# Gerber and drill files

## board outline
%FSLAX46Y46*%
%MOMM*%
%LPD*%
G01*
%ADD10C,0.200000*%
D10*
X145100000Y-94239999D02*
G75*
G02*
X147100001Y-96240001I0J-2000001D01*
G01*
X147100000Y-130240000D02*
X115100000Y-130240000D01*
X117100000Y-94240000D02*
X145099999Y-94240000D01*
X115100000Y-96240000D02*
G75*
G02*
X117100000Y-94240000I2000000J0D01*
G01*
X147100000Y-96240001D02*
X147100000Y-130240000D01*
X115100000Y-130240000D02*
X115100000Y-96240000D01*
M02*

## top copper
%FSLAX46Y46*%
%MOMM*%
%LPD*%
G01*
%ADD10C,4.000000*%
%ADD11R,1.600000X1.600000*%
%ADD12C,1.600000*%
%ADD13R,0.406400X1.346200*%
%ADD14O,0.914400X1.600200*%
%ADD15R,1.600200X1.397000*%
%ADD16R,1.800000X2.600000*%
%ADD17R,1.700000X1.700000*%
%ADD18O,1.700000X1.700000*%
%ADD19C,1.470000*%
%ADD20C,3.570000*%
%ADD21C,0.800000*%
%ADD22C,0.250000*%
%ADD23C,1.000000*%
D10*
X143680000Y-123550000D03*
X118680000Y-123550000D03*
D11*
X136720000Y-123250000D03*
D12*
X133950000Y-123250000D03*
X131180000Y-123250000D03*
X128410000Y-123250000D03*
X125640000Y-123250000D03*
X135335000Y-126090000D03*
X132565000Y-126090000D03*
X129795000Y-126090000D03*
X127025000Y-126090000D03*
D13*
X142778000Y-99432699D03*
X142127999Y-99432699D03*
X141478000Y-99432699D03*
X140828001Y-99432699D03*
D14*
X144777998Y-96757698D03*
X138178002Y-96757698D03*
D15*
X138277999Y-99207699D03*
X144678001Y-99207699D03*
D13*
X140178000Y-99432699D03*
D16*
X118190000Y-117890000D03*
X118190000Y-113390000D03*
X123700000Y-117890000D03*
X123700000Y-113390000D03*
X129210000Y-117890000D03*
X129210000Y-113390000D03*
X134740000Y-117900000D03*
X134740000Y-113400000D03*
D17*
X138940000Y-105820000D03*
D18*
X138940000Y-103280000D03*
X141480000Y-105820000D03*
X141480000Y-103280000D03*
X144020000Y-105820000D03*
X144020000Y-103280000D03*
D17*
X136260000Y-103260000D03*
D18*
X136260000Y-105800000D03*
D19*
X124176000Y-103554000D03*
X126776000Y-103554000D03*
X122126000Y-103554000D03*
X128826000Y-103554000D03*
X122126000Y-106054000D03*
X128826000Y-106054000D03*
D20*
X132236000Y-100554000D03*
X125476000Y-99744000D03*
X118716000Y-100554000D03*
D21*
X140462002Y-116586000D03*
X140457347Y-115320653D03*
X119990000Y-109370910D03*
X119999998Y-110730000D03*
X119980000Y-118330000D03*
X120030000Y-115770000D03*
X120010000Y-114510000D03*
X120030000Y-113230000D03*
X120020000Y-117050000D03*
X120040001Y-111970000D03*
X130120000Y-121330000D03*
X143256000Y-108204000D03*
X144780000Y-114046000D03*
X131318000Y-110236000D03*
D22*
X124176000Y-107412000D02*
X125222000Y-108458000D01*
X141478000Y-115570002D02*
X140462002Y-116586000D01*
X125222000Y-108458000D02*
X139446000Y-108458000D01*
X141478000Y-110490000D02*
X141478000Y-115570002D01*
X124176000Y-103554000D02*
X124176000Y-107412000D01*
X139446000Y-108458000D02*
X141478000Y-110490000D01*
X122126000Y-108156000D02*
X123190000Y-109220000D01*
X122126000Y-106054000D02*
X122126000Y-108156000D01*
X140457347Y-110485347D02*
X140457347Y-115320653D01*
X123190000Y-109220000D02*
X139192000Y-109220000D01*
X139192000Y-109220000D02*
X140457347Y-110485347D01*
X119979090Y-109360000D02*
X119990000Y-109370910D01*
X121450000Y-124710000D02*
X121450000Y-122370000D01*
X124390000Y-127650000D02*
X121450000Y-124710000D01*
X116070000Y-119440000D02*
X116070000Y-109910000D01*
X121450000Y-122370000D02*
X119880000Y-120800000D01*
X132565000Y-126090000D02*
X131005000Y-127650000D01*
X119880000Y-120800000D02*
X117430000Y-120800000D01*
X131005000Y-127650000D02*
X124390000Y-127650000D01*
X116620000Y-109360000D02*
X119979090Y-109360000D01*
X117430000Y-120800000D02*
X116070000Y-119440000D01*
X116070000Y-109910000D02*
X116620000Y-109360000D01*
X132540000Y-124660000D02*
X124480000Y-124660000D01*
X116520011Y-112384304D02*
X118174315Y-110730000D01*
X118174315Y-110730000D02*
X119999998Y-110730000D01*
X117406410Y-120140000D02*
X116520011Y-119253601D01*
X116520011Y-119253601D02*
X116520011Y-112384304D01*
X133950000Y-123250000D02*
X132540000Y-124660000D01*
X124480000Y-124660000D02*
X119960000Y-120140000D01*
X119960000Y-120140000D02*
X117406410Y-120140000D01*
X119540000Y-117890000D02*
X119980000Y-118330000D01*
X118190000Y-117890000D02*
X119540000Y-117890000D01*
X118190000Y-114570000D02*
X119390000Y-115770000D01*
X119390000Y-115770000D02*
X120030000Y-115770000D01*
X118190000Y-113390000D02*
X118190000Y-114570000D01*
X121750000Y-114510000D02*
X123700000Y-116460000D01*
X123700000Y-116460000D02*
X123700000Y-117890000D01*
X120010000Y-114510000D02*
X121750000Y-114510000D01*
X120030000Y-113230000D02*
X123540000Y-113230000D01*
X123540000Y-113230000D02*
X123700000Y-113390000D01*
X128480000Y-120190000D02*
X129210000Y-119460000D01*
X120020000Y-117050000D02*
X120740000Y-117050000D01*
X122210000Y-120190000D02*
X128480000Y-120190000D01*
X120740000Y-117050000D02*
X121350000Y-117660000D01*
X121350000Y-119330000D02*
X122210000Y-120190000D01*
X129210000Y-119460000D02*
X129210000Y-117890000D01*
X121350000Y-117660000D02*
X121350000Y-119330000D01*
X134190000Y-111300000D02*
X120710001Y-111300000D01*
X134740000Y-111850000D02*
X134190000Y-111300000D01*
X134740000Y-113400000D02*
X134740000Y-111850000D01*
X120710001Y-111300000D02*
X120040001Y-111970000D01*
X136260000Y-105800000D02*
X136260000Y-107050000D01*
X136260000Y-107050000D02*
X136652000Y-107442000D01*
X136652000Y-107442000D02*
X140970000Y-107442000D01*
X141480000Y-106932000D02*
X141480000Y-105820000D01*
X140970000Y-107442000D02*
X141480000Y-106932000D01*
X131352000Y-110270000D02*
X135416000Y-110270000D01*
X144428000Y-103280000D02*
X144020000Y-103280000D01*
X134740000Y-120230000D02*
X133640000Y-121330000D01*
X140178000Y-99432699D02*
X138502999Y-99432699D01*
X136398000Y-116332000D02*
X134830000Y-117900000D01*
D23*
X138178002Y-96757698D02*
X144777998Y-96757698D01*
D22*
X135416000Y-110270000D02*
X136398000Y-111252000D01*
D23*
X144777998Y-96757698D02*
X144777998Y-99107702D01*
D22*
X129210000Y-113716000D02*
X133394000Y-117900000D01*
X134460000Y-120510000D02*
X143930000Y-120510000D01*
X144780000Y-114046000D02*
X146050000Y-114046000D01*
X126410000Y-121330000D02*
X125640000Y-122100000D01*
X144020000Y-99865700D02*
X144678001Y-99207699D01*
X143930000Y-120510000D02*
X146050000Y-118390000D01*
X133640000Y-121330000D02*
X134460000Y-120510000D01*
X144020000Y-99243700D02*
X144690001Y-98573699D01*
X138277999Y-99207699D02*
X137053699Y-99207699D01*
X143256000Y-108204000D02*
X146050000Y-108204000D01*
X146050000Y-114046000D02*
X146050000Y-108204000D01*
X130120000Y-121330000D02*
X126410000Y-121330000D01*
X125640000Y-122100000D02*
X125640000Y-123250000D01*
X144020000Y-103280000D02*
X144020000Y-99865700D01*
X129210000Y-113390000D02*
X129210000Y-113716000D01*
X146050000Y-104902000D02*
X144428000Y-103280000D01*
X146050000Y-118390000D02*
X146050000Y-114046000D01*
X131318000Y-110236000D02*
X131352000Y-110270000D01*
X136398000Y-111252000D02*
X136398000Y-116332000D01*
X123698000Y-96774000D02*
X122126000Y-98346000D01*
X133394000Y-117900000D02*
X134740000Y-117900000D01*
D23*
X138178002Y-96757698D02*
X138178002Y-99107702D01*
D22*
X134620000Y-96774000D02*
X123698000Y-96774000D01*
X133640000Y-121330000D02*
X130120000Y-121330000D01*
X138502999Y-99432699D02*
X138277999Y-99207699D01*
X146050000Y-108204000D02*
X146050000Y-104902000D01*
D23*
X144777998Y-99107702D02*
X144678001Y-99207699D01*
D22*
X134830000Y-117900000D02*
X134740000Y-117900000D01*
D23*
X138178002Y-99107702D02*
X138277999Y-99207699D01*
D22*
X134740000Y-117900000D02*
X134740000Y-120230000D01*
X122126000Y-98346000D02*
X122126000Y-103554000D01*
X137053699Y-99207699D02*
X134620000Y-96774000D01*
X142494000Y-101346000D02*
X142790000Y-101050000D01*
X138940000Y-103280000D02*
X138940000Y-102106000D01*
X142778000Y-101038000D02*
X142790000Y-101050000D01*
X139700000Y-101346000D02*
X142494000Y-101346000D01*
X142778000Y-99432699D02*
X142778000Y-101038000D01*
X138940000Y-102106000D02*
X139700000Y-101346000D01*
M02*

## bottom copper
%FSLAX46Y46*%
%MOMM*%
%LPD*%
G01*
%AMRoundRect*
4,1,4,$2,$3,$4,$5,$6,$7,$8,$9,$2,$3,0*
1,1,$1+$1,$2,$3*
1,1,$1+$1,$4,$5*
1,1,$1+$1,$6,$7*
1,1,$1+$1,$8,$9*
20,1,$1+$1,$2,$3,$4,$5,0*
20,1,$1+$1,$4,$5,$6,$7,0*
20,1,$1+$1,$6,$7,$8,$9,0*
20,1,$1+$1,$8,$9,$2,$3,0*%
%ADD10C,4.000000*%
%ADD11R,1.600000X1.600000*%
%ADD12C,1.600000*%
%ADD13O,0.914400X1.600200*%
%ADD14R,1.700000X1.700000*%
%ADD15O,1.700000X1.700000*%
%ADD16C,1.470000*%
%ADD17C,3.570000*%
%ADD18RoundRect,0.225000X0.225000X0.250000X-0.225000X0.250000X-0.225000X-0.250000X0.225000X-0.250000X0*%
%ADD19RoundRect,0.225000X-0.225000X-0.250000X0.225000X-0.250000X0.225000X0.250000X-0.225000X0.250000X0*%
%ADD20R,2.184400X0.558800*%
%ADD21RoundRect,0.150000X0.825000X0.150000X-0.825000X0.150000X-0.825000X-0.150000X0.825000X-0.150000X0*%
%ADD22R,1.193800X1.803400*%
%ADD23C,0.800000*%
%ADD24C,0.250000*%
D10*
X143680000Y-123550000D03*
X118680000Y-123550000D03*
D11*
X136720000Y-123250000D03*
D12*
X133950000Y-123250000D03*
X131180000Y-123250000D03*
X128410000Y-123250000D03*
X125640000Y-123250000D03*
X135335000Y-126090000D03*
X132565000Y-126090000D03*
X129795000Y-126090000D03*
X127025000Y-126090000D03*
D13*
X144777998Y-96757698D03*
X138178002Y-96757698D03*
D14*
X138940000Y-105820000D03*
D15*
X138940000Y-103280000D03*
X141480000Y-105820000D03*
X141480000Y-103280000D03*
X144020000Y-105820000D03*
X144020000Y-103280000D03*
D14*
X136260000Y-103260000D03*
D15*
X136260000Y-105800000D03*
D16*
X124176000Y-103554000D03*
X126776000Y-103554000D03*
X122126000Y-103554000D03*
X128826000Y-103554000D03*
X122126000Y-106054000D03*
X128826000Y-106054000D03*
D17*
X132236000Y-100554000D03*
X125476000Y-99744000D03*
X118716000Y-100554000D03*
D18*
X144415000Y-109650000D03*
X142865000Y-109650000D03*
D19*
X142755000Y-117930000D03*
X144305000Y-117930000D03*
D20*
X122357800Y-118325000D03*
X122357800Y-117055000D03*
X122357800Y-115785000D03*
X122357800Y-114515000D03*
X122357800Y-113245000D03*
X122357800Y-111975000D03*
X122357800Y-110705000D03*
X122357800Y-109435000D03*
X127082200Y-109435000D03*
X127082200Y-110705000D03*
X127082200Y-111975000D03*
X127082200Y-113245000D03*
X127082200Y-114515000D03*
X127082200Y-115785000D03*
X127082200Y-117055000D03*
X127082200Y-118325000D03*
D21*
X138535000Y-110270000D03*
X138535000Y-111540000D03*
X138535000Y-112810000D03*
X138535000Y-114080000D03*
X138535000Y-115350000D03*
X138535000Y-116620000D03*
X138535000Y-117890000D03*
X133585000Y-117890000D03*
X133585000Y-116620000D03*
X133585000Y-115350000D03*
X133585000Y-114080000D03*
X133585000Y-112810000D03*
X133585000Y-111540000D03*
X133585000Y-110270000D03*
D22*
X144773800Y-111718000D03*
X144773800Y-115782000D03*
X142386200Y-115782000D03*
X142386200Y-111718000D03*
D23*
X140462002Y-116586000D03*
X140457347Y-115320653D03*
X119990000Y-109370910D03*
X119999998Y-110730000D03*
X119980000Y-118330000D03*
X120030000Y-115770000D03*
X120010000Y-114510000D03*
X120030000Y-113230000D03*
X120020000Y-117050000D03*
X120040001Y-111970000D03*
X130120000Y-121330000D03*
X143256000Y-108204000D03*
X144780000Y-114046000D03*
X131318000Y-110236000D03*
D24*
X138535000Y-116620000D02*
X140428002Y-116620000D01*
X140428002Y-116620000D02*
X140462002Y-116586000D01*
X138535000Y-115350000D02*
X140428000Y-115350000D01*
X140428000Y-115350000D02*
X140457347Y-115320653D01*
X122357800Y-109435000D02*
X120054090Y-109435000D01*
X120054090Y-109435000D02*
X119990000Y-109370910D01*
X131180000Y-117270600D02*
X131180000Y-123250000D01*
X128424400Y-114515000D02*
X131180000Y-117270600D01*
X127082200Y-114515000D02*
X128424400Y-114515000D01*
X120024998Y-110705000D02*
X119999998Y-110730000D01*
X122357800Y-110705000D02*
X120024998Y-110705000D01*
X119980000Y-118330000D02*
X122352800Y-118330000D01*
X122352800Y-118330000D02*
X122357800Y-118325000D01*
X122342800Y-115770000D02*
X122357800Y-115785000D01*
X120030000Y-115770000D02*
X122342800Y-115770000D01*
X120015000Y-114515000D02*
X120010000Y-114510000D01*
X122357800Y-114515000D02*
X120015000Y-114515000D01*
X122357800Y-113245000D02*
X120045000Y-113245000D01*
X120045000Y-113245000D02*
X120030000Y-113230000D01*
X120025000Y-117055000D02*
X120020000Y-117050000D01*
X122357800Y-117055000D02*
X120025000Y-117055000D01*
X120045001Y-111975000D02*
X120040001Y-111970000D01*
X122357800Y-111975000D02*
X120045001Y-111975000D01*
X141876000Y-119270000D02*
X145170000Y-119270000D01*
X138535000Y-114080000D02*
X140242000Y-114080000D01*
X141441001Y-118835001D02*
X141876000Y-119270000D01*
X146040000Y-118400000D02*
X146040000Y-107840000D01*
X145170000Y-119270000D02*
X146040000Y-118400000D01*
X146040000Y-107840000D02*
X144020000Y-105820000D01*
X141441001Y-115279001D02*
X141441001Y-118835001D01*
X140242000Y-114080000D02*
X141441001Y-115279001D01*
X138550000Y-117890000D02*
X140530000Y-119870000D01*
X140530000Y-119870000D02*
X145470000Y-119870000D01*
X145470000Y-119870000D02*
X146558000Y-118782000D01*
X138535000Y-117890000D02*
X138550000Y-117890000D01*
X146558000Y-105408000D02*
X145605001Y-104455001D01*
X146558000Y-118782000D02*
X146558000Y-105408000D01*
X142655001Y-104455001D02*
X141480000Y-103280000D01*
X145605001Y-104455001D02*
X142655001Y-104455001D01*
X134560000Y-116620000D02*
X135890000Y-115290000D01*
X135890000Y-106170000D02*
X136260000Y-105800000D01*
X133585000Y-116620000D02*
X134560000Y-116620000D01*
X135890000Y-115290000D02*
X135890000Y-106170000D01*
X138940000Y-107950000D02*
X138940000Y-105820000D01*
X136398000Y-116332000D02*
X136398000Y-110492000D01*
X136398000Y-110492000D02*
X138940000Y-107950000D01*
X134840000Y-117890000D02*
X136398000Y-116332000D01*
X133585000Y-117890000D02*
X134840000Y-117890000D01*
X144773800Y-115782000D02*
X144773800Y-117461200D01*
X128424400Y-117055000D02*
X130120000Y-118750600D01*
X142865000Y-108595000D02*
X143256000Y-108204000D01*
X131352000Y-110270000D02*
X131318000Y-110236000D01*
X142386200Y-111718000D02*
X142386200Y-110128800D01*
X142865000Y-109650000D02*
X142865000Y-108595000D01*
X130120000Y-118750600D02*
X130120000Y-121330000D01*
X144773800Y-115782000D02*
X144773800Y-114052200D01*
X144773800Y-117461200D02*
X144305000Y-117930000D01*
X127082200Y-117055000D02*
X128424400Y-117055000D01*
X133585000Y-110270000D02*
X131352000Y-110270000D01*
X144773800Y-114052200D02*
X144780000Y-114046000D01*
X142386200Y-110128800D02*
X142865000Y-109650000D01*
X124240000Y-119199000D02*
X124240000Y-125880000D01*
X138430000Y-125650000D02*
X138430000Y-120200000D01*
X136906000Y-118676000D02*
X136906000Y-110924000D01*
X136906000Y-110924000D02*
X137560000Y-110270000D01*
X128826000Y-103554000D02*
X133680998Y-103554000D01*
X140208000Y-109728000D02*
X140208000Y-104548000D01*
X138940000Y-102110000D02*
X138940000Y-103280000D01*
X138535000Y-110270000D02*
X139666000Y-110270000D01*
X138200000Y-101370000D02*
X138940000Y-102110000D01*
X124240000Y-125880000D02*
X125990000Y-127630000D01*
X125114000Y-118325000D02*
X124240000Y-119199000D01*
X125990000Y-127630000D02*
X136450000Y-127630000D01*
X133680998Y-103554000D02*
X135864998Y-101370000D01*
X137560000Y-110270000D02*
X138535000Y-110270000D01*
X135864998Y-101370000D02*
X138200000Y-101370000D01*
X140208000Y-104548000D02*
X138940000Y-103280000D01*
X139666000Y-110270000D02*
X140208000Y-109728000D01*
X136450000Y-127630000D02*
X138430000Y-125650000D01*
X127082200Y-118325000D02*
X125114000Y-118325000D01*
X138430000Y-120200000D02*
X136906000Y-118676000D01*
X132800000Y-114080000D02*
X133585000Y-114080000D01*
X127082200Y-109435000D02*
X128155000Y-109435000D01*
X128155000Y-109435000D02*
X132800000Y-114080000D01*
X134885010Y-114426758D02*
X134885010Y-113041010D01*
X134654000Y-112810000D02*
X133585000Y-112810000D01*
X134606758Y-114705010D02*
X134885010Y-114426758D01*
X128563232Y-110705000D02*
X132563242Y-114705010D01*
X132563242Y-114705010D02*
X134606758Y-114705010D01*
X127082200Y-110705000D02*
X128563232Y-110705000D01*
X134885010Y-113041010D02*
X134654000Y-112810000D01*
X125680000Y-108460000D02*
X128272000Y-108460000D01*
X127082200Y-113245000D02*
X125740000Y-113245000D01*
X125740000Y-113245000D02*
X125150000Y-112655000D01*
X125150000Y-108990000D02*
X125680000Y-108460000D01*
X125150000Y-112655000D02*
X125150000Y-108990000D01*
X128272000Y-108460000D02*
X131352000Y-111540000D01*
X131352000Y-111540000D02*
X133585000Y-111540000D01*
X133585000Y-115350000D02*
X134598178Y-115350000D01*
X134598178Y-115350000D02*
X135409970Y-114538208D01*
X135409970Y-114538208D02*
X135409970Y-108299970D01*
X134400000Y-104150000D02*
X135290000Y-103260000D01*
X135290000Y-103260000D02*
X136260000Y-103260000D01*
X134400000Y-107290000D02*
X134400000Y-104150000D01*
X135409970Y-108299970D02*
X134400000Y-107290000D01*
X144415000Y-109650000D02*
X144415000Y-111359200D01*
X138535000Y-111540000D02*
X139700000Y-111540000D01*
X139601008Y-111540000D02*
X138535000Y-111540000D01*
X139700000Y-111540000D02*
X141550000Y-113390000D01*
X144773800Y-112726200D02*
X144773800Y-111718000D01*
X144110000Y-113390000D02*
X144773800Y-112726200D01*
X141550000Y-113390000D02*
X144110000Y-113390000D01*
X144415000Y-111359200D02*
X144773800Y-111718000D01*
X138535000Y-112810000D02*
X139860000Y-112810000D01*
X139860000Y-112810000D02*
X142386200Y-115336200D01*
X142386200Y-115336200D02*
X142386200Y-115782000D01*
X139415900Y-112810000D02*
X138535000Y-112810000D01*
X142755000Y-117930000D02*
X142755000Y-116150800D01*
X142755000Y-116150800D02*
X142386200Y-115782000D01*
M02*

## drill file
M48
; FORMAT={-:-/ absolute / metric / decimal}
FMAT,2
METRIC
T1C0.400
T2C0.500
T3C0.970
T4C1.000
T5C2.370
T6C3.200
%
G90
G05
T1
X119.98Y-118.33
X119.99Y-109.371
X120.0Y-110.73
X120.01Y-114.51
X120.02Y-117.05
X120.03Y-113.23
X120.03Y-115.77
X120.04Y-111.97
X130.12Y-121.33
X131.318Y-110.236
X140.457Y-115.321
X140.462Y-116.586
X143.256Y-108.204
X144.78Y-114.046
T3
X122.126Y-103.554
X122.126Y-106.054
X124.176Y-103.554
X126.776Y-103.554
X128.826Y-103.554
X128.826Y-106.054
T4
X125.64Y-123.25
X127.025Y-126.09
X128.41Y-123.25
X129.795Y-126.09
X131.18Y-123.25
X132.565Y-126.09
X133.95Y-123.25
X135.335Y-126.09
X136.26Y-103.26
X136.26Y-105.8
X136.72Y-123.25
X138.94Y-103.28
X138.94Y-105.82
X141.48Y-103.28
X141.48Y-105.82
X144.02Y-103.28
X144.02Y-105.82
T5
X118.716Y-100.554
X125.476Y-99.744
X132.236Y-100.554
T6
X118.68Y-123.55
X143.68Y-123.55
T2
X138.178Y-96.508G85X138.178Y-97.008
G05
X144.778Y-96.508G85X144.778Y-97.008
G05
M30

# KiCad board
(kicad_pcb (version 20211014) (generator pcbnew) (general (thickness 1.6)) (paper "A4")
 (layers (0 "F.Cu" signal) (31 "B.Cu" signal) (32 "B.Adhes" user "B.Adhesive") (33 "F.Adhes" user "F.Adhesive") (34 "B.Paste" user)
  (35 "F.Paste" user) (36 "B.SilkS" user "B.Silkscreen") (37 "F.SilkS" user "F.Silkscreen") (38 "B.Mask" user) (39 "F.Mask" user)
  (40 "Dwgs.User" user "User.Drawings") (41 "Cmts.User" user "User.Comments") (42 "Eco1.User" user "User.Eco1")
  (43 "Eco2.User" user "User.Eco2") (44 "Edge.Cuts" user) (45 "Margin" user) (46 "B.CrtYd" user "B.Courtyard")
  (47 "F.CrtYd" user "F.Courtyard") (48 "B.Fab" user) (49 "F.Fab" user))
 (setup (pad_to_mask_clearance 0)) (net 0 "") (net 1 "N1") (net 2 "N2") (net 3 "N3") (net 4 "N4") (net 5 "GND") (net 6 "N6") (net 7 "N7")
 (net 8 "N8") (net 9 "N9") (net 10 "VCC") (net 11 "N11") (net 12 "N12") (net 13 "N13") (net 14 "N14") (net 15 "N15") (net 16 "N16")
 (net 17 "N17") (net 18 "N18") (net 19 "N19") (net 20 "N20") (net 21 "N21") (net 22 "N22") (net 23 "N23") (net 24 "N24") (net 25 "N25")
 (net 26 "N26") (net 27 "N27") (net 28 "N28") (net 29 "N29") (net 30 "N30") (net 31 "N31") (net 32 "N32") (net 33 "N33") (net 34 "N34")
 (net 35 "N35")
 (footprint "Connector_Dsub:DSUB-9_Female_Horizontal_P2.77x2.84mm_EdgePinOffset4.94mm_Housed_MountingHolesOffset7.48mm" (layer "F.Cu")
  (at 136.72 123.25)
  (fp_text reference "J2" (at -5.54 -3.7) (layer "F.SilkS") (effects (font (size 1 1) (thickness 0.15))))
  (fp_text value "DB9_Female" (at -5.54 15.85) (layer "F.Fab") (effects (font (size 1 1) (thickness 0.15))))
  (pad "0" thru_hole circle locked (at 6.96 0.3) (size 4 4) (drill 3.2) (layers *.Cu *.Mask))
  (pad "0" thru_hole circle locked (at -18.04 0.3) (size 4 4) (drill 3.2) (layers *.Cu *.Mask))
  (pad "1" thru_hole rect locked (at 0 0) (size 1.6 1.6) (drill 1) (layers *.Cu *.Mask) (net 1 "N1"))
  (pad "2" thru_hole circle locked (at -2.77 0) (size 1.6 1.6) (drill 1) (layers *.Cu *.Mask) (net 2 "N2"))
  (pad "3" thru_hole circle locked (at -5.54 0) (size 1.6 1.6) (drill 1) (layers *.Cu *.Mask) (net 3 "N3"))
  (pad "4" thru_hole circle locked (at -8.31 0) (size 1.6 1.6) (drill 1) (layers *.Cu *.Mask) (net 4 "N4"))
  (pad "5" thru_hole circle locked (at -11.08 0) (size 1.6 1.6) (drill 1) (layers *.Cu *.Mask) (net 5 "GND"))
  (pad "6" thru_hole circle locked (at -1.385 2.84) (size 1.6 1.6) (drill 1) (layers *.Cu *.Mask) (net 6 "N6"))
  (pad "7" thru_hole circle locked (at -4.155 2.84) (size 1.6 1.6) (drill 1) (layers *.Cu *.Mask) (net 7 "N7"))
  (pad "8" thru_hole circle locked (at -6.925 2.84) (size 1.6 1.6) (drill 1) (layers *.Cu *.Mask) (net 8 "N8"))
  (pad "9" thru_hole circle locked (at -9.695 2.84) (size 1.6 1.6) (drill 1) (layers *.Cu *.Mask) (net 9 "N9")))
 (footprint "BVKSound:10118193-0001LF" (layer "F.Cu") (at 141.478 96.774 180)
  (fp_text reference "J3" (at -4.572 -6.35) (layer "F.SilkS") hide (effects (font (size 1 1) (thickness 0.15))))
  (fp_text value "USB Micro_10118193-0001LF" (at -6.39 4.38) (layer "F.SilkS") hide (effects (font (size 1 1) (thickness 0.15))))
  (pad "1" smd rect locked (at -1.3 -2.658699 180) (size 0.4064 1.3462) (layers "F.Cu" "F.Paste" "F.Mask") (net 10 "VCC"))
  (pad "2" smd rect locked (at -0.649999 -2.658699 180) (size 0.4064 1.3462) (layers "F.Cu" "F.Paste" "F.Mask") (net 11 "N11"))
  (pad "3" smd rect locked (at 0 -2.658699 180) (size 0.4064 1.3462) (layers "F.Cu" "F.Paste" "F.Mask") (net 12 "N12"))
  (pad "4" smd rect locked (at 0.649999 -2.658699 180) (size 0.4064 1.3462) (layers "F.Cu" "F.Paste" "F.Mask") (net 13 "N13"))
  (pad "5" thru_hole oval locked (at -3.299998 0.016302 270) (size 1.6002 0.9144) (drill oval 1 0.5) (layers *.Cu *.Mask) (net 5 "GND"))
  (pad "5" thru_hole oval locked (at 3.299998 0.016302 270) (size 1.6002 0.9144) (drill oval 1 0.5) (layers *.Cu *.Mask) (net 5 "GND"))
  (pad "5" smd rect locked (at 3.200001 -2.433699 180) (size 1.6002 1.397) (layers "F.Cu" "F.Paste" "F.Mask") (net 5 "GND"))
  (pad "5" smd rect locked (at -3.200001 -2.433699 180) (size 1.6002 1.397) (layers "F.Cu" "F.Paste" "F.Mask") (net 5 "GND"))
  (pad "5" smd rect locked (at 1.3 -2.658699 180) (size 0.4064 1.3462) (layers "F.Cu" "F.Paste" "F.Mask") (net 5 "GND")))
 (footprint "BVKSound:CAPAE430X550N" (layer "F.Cu") (at 118.19 115.64 90)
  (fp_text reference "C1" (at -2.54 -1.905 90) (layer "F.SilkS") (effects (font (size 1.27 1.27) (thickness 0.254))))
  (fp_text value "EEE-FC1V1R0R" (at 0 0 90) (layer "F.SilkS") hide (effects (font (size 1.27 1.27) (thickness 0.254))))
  (pad "1" smd rect locked (at -2.25 0 180) (size 1.8 2.6) (layers "F.Cu" "F.Paste" "F.Mask") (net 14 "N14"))
  (pad "2" smd rect locked (at 2.25 0 180) (size 1.8 2.6) (layers "F.Cu" "F.Paste" "F.Mask") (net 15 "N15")))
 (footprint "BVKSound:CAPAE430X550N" (layer "F.Cu") (at 123.7 115.64 90)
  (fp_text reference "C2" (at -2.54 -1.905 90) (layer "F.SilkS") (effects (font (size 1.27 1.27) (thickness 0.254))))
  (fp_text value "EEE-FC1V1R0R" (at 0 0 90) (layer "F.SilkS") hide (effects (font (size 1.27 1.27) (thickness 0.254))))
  (pad "1" smd rect locked (at -2.25 0 180) (size 1.8 2.6) (layers "F.Cu" "F.Paste" "F.Mask") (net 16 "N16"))
  (pad "2" smd rect locked (at 2.25 0 180) (size 1.8 2.6) (layers "F.Cu" "F.Paste" "F.Mask") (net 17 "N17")))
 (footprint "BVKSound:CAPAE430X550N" (layer "F.Cu") (at 129.21 115.64 90)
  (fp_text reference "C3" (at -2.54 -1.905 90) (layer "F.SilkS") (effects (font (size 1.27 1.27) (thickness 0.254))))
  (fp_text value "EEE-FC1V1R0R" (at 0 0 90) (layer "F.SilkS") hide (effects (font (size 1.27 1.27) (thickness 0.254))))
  (pad "1" smd rect locked (at -2.25 0 180) (size 1.8 2.6) (layers "F.Cu" "F.Paste" "F.Mask") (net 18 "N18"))
  (pad "2" smd rect locked (at 2.25 0 180) (size 1.8 2.6) (layers "F.Cu" "F.Paste" "F.Mask") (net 5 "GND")))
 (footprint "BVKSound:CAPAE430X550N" (layer "F.Cu") (at 134.74 115.65 90)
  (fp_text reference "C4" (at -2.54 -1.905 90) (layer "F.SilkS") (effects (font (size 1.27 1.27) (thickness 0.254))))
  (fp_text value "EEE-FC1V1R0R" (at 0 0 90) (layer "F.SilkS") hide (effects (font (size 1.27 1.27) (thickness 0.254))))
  (pad "1" smd rect locked (at -2.25 0 180) (size 1.8 2.6) (layers "F.Cu" "F.Paste" "F.Mask") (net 5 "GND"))
  (pad "2" smd rect locked (at 2.25 0 180) (size 1.8 2.6) (layers "F.Cu" "F.Paste" "F.Mask") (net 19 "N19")))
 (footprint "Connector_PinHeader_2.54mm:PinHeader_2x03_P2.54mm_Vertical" (layer "F.Cu") (at 138.94 105.82 90)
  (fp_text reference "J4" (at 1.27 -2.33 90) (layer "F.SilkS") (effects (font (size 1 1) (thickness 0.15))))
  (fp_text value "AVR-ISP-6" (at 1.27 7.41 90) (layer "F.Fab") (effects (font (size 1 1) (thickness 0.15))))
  (pad "1" thru_hole rect locked (at 0 0 90) (size 1.7 1.7) (drill 1) (layers *.Cu *.Mask) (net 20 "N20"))
  (pad "2" thru_hole oval locked (at 2.54 0 90) (size 1.7 1.7) (drill 1) (layers *.Cu *.Mask) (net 10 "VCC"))
  (pad "3" thru_hole oval locked (at 0 2.54 90) (size 1.7 1.7) (drill 1) (layers *.Cu *.Mask) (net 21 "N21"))
  (pad "4" thru_hole oval locked (at 2.54 2.54 90) (size 1.7 1.7) (drill 1) (layers *.Cu *.Mask) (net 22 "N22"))
  (pad "5" thru_hole oval locked (at 0 5.08 90) (size 1.7 1.7) (drill 1) (layers *.Cu *.Mask) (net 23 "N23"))
  (pad "6" thru_hole oval locked (at 2.54 5.08 90) (size 1.7 1.7) (drill 1) (layers *.Cu *.Mask) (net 5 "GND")))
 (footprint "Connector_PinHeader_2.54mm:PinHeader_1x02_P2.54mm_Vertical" (layer "F.Cu") (at 136.26 103.26)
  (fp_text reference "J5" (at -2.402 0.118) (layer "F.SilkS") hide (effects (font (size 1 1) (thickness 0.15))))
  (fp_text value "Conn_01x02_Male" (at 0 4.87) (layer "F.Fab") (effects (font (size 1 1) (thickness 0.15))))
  (pad "1" thru_hole rect locked (at 0 0) (size 1.7 1.7) (drill 1) (layers *.Cu *.Mask) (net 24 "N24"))
  (pad "2" thru_hole oval locked (at 0 2.54) (size 1.7 1.7) (drill 1) (layers *.Cu *.Mask) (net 21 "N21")))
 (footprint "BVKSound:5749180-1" (layer "B.Cu") (at 125.476 94.234 180)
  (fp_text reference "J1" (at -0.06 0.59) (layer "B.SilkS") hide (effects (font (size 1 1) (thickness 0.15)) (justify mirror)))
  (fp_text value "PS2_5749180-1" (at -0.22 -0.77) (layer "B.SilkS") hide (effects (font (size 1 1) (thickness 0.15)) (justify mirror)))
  (pad "1" thru_hole circle locked (at 1.3 -9.32 180) (size 1.47 1.47) (drill 0.97) (layers *.Cu *.Mask) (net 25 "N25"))
  (pad "2" thru_hole circle locked (at -1.3 -9.32 180) (size 1.47 1.47) (drill 0.97) (layers *.Cu *.Mask) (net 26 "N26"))
  (pad "3" thru_hole circle locked (at 3.35 -9.32 180) (size 1.47 1.47) (drill 0.97) (layers *.Cu *.Mask) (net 5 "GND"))
  (pad "4" thru_hole circle locked (at -3.35 -9.32 180) (size 1.47 1.47) (drill 0.97) (layers *.Cu *.Mask) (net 10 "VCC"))
  (pad "5" thru_hole circle locked (at 3.35 -11.82 180) (size 1.47 1.47) (drill 0.97) (layers *.Cu *.Mask) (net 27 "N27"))
  (pad "6" thru_hole circle locked (at -3.35 -11.82 180) (size 1.47 1.47) (drill 0.97) (layers *.Cu *.Mask) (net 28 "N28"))
  (pad "7" thru_hole circle locked (at -6.76 -6.32 180) (size 3.57 3.57) (drill 2.37) (layers *.Cu *.Mask))
  (pad "8" thru_hole circle locked (at 0 -5.51 180) (size 3.57 3.57) (drill 2.37) (layers *.Cu *.Mask))
  (pad "9" thru_hole circle locked (at 6.76 -6.32 180) (size 3.57 3.57) (drill 2.37) (layers *.Cu *.Mask)))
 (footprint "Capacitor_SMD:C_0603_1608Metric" (layer "B.Cu") (at 143.64 109.65 180)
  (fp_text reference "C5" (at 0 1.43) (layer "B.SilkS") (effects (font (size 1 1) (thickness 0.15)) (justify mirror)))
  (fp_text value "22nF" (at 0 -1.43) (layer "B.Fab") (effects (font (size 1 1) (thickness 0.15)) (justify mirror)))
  (pad "1" smd roundrect locked (at -0.775 0 180) (size 0.9 0.95) (layers "B.Cu" "B.Paste" "B.Mask") (roundrect_rratio 0.25) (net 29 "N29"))
  (pad "2" smd roundrect locked (at 0.775 0 180) (size 0.9 0.95) (layers "B.Cu" "B.Paste" "B.Mask") (roundrect_rratio 0.25) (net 5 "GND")))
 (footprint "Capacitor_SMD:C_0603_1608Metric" (layer "B.Cu") (at 143.53 117.93)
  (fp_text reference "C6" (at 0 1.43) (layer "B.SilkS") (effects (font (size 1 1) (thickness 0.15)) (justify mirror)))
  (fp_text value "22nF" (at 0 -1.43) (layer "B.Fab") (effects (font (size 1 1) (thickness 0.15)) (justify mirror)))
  (pad "1" smd roundrect locked (at -0.775 0) (size 0.9 0.95) (layers "B.Cu" "B.Paste" "B.Mask") (roundrect_rratio 0.25) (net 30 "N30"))
  (pad "2" smd roundrect locked (at 0.775 0) (size 0.9 0.95) (layers "B.Cu" "B.Paste" "B.Mask") (roundrect_rratio 0.25) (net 5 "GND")))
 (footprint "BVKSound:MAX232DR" (layer "B.Cu") (at 124.72 113.88)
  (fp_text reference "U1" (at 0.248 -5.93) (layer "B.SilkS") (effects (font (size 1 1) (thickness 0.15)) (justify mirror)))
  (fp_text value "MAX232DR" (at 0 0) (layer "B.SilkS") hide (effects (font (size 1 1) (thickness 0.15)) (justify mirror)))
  (pad "1" smd rect locked (at -2.3622 4.445) (size 2.1844 0.5588) (layers "B.Cu" "B.Paste" "B.Mask") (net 14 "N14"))
  (pad "2" smd rect locked (at -2.3622 3.175) (size 2.1844 0.5588) (layers "B.Cu" "B.Paste" "B.Mask") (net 18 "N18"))
  (pad "3" smd rect locked (at -2.3622 1.905) (size 2.1844 0.5588) (layers "B.Cu" "B.Paste" "B.Mask") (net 15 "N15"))
  (pad "4" smd rect locked (at -2.3622 0.635) (size 2.1844 0.5588) (layers "B.Cu" "B.Paste" "B.Mask") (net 16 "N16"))
  (pad "5" smd rect locked (at -2.3622 -0.635) (size 2.1844 0.5588) (layers "B.Cu" "B.Paste" "B.Mask") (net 17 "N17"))
  (pad "6" smd rect locked (at -2.3622 -1.905) (size 2.1844 0.5588) (layers "B.Cu" "B.Paste" "B.Mask") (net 19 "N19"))
  (pad "7" smd rect locked (at -2.3622 -3.175) (size 2.1844 0.5588) (layers "B.Cu" "B.Paste" "B.Mask") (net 2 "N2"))
  (pad "8" smd rect locked (at -2.3622 -4.445) (size 2.1844 0.5588) (layers "B.Cu" "B.Paste" "B.Mask") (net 7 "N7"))
  (pad "9" smd rect locked (at 2.3622 -4.445) (size 2.1844 0.5588) (layers "B.Cu" "B.Paste" "B.Mask") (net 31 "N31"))
  (pad "10" smd rect locked (at 2.3622 -3.175) (size 2.1844 0.5588) (layers "B.Cu" "B.Paste" "B.Mask") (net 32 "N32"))
  (pad "11" smd rect locked (at 2.3622 -1.905) (size 2.1844 0.5588) (layers "B.Cu" "B.Paste" "B.Mask") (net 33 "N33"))
  (pad "12" smd rect locked (at 2.3622 -0.635) (size 2.1844 0.5588) (layers "B.Cu" "B.Paste" "B.Mask") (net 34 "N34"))
  (pad "13" smd rect locked (at 2.3622 0.635) (size 2.1844 0.5588) (layers "B.Cu" "B.Paste" "B.Mask") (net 3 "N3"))
  (pad "14" smd rect locked (at 2.3622 1.905) (size 2.1844 0.5588) (layers "B.Cu" "B.Paste" "B.Mask") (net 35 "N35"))
  (pad "15" smd rect locked (at 2.3622 3.175) (size 2.1844 0.5588) (layers "B.Cu" "B.Paste" "B.Mask") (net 5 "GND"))
  (pad "16" smd rect locked (at 2.3622 4.445) (size 2.1844 0.5588) (layers "B.Cu" "B.Paste" "B.Mask") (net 10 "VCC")))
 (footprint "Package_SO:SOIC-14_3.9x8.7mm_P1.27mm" (layer "B.Cu") (at 136.06 114.08 180)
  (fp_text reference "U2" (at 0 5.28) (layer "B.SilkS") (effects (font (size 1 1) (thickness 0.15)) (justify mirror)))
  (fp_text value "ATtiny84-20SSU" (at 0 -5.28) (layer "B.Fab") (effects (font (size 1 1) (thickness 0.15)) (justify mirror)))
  (pad "1" smd roundrect locked (at -2.475 3.81 180) (size 1.95 0.6) (layers "B.Cu" "B.Paste" "B.Mask") (roundrect_rratio 0.25)
   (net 10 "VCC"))
  (pad "2" smd roundrect locked (at -2.475 2.54 180) (size 1.95 0.6) (layers "B.Cu" "B.Paste" "B.Mask") (roundrect_rratio 0.25)
   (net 29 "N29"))
  (pad "3" smd roundrect locked (at -2.475 1.27 180) (size 1.95 0.6) (layers "B.Cu" "B.Paste" "B.Mask") (roundrect_rratio 0.25)
   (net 30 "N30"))
  (pad "4" smd roundrect locked (at -2.475 0 180) (size 1.95 0.6) (layers "B.Cu" "B.Paste" "B.Mask") (roundrect_rratio 0.25) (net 23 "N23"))
  (pad "5" smd roundrect locked (at -2.475 -1.27 180) (size 1.95 0.6) (layers "B.Cu" "B.Paste" "B.Mask") (roundrect_rratio 0.25)
   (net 27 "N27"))
  (pad "6" smd roundrect locked (at -2.475 -2.54 180) (size 1.95 0.6) (layers "B.Cu" "B.Paste" "B.Mask") (roundrect_rratio 0.25)
   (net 25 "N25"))
  (pad "7" smd roundrect locked (at -2.475 -3.81 180) (size 1.95 0.6) (layers "B.Cu" "B.Paste" "B.Mask") (roundrect_rratio 0.25)
   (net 22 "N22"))
  (pad "8" smd roundrect locked (at 2.475 -3.81 180) (size 1.95 0.6) (layers "B.Cu" "B.Paste" "B.Mask") (roundrect_rratio 0.25)
   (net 20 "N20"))
  (pad "9" smd roundrect locked (at 2.475 -2.54 180) (size 1.95 0.6) (layers "B.Cu" "B.Paste" "B.Mask") (roundrect_rratio 0.25)
   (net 21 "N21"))
  (pad "10" smd roundrect locked (at 2.475 -1.27 180) (size 1.95 0.6) (layers "B.Cu" "B.Paste" "B.Mask") (roundrect_rratio 0.25)
   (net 24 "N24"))
  (pad "11" smd roundrect locked (at 2.475 0 180) (size 1.95 0.6) (layers "B.Cu" "B.Paste" "B.Mask") (roundrect_rratio 0.25) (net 31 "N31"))
  (pad "12" smd roundrect locked (at 2.475 1.27 180) (size 1.95 0.6) (layers "B.Cu" "B.Paste" "B.Mask") (roundrect_rratio 0.25)
   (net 32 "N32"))
  (pad "13" smd roundrect locked (at 2.475 2.54 180) (size 1.95 0.6) (layers "B.Cu" "B.Paste" "B.Mask") (roundrect_rratio 0.25)
   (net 34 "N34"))
  (pad "14" smd roundrect locked (at 2.475 3.81 180) (size 1.95 0.6) (layers "B.Cu" "B.Paste" "B.Mask") (roundrect_rratio 0.25)
   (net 5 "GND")))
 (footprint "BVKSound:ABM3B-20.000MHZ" (layer "B.Cu") (at 143.58 113.75 180)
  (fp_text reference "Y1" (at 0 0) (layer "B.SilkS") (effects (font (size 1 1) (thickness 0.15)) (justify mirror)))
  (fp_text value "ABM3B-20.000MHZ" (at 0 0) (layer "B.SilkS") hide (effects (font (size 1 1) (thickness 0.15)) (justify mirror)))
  (pad "1" smd rect locked (at -1.1938 2.032 180) (size 1.1938 1.8034) (layers "B.Cu" "B.Paste" "B.Mask") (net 29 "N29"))
  (pad "2" smd rect locked (at -1.1938 -2.032 180) (size 1.1938 1.8034) (layers "B.Cu" "B.Paste" "B.Mask") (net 5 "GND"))
  (pad "3" smd rect locked (at 1.1938 -2.032 180) (size 1.1938 1.8034) (layers "B.Cu" "B.Paste" "B.Mask") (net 30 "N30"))
  (pad "4" smd rect locked (at 1.1938 2.032 180) (size 1.1938 1.8034) (layers "B.Cu" "B.Paste" "B.Mask") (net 5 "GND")))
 (gr_arc (start 145.1 94.239999) (mid 146.514214 94.825786) (end 147.1 96.240001) (layer "Edge.Cuts") (width 0.2))
 (gr_line (start 147.1 130.24) (end 115.1 130.24) (layer "Edge.Cuts") (width 0.2))
 (gr_line (start 117.1 94.24) (end 145.099999 94.24) (layer "Edge.Cuts") (width 0.2))
 (gr_arc (start 115.1 96.24) (mid 115.685786 94.825786) (end 117.1 94.24) (layer "Edge.Cuts") (width 0.2))
 (gr_line (start 147.1 96.240001) (end 147.1 130.24) (layer "Edge.Cuts") (width 0.2))
 (gr_line (start 115.1 130.24) (end 115.1 96.24) (layer "Edge.Cuts") (width 0.2))
 (segment (start 124.176 107.412) (end 125.222 108.458) (width 0.25) (layer "F.Cu") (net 25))
 (segment (start 141.478 115.570002) (end 140.462002 116.586) (width 0.25) (layer "F.Cu") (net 25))
 (segment (start 125.222 108.458) (end 139.446 108.458) (width 0.25) (layer "F.Cu") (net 25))
 (segment (start 141.478 110.49) (end 141.478 115.570002) (width 0.25) (layer "F.Cu") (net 25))
 (segment (start 124.176 103.554) (end 124.176 107.412) (width 0.25) (layer "F.Cu") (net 25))
 (segment (start 139.446 108.458) (end 141.478 110.49) (width 0.25) (layer "F.Cu") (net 25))
 (via (at 140.462002 116.586) (size 0.8) (drill 0.4) (layers "F.Cu" "B.Cu") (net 25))
 (segment (start 138.535 116.62) (end 140.428002 116.62) (width 0.25) (layer "B.Cu") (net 25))
 (segment (start 140.428002 116.62) (end 140.462002 116.586) (width 0.25) (layer "B.Cu") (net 25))
 (segment (start 122.126 108.156) (end 123.19 109.22) (width 0.25) (layer "F.Cu") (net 27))
 (segment (start 122.126 106.054) (end 122.126 108.156) (width 0.25) (layer "F.Cu") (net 27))
 (segment (start 140.457347 110.485347) (end 140.457347 115.320653) (width 0.25) (layer "F.Cu") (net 27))
 (segment (start 123.19 109.22) (end 139.192 109.22) (width 0.25) (layer "F.Cu") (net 27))
 (segment (start 139.192 109.22) (end 140.457347 110.485347) (width 0.25) (layer "F.Cu") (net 27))
 (via (at 140.457347 115.320653) (size 0.8) (drill 0.4) (layers "F.Cu" "B.Cu") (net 27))
 (segment (start 138.535 115.35) (end 140.428 115.35) (width 0.25) (layer "B.Cu") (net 27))
 (segment (start 140.428 115.35) (end 140.457347 115.320653) (width 0.25) (layer "B.Cu") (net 27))
 (segment (start 119.97909 109.36) (end 119.99 109.37091) (width 0.25) (layer "F.Cu") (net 7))
 (segment (start 121.45 124.71) (end 121.45 122.37) (width 0.25) (layer "F.Cu") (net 7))
 (segment (start 124.39 127.65) (end 121.45 124.71) (width 0.25) (layer "F.Cu") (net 7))
 (segment (start 116.07 119.44) (end 116.07 109.91) (width 0.25) (layer "F.Cu") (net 7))
 (segment (start 121.45 122.37) (end 119.88 120.8) (width 0.25) (layer "F.Cu") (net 7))
 (segment (start 132.565 126.09) (end 131.005 127.65) (width 0.25) (layer "F.Cu") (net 7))
 (segment (start 119.88 120.8) (end 117.43 120.8) (width 0.25) (layer "F.Cu") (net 7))
 (segment (start 131.005 127.65) (end 124.39 127.65) (width 0.25) (layer "F.Cu") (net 7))
 (segment (start 116.62 109.36) (end 119.97909 109.36) (width 0.25) (layer "F.Cu") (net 7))
 (segment (start 117.43 120.8) (end 116.07 119.44) (width 0.25) (layer "F.Cu") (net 7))
 (segment (start 116.07 109.91) (end 116.62 109.36) (width 0.25) (layer "F.Cu") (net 7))
 (via (at 119.99 109.37091) (size 0.8) (drill 0.4) (layers "F.Cu" "B.Cu") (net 7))
 (segment (start 122.3578 109.435) (end 120.05409 109.435) (width 0.25) (layer "B.Cu") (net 7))
 (segment (start 120.05409 109.435) (end 119.99 109.37091) (width 0.25) (layer "B.Cu") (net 7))
 (segment (start 131.18 117.2706) (end 131.18 123.25) (width 0.25) (layer "B.Cu") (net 3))
 (segment (start 128.4244 114.515) (end 131.18 117.2706) (width 0.25) (layer "B.Cu") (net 3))
 (segment (start 127.0822 114.515) (end 128.4244 114.515) (width 0.25) (layer "B.Cu") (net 3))
 (segment (start 132.54 124.66) (end 124.48 124.66) (width 0.25) (layer "F.Cu") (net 2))
 (segment (start 116.520011 112.384304) (end 118.174315 110.73) (width 0.25) (layer "F.Cu") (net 2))
 (segment (start 118.174315 110.73) (end 119.999998 110.73) (width 0.25) (layer "F.Cu") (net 2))
 (segment (start 117.40641 120.14) (end 116.520011 119.253601) (width 0.25) (layer "F.Cu") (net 2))
 (segment (start 116.520011 119.253601) (end 116.520011 112.384304) (width 0.25) (layer "F.Cu") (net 2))
 (segment (start 133.95 123.25) (end 132.54 124.66) (width 0.25) (layer "F.Cu") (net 2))
 (segment (start 124.48 124.66) (end 119.96 120.14) (width 0.25) (layer "F.Cu") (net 2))
 (segment (start 119.96 120.14) (end 117.40641 120.14) (width 0.25) (layer "F.Cu") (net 2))
 (via (at 119.999998 110.73) (size 0.8) (drill 0.4) (layers "F.Cu" "B.Cu") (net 2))
 (segment (start 120.024998 110.705) (end 119.999998 110.73) (width 0.25) (layer "B.Cu") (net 2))
 (segment (start 122.3578 110.705) (end 120.024998 110.705) (width 0.25) (layer "B.Cu") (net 2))
 (segment (start 119.54 117.89) (end 119.98 118.33) (width 0.25) (layer "F.Cu") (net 14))
 (segment (start 118.19 117.89) (end 119.54 117.89) (width 0.25) (layer "F.Cu") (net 14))
 (via (at 119.98 118.33) (size 0.8) (drill 0.4) (layers "F.Cu" "B.Cu") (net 14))
 (segment (start 119.98 118.33) (end 122.3528 118.33) (width 0.25) (layer "B.Cu") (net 14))
 (segment (start 122.3528 118.33) (end 122.3578 118.325) (width 0.25) (layer "B.Cu") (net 14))
 (segment (start 118.19 114.57) (end 119.39 115.77) (width 0.25) (layer "F.Cu") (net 15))
 (segment (start 119.39 115.77) (end 120.03 115.77) (width 0.25) (layer "F.Cu") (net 15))
 (segment (start 118.19 113.39) (end 118.19 114.57) (width 0.25) (layer "F.Cu") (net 15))
 (via (at 120.03 115.77) (size 0.8) (drill 0.4) (layers "F.Cu" "B.Cu") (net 15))
 (segment (start 122.3428 115.77) (end 122.3578 115.785) (width 0.25) (layer "B.Cu") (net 15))
 (segment (start 120.03 115.77) (end 122.3428 115.77) (width 0.25) (layer "B.Cu") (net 15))
 (segment (start 121.75 114.51) (end 123.7 116.46) (width 0.25) (layer "F.Cu") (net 16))
 (segment (start 123.7 116.46) (end 123.7 117.89) (width 0.25) (layer "F.Cu") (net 16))
 (segment (start 120.01 114.51) (end 121.75 114.51) (width 0.25) (layer "F.Cu") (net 16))
 (via (at 120.01 114.51) (size 0.8) (drill 0.4) (layers "F.Cu" "B.Cu") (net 16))
 (segment (start 120.015 114.515) (end 120.01 114.51) (width 0.25) (layer "B.Cu") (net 16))
 (segment (start 122.3578 114.515) (end 120.015 114.515) (width 0.25) (layer "B.Cu") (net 16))
 (segment (start 120.03 113.23) (end 123.54 113.23) (width 0.25) (layer "F.Cu") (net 17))
 (segment (start 123.54 113.23) (end 123.7 113.39) (width 0.25) (layer "F.Cu") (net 17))
 (via (at 120.03 113.23) (size 0.8) (drill 0.4) (layers "F.Cu" "B.Cu") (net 17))
 (segment (start 122.3578 113.245) (end 120.045 113.245) (width 0.25) (layer "B.Cu") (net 17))
 (segment (start 120.045 113.245) (end 120.03 113.23) (width 0.25) (layer "B.Cu") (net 17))
 (segment (start 128.48 120.19) (end 129.21 119.46) (width 0.25) (layer "F.Cu") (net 18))
 (segment (start 120.02 117.05) (end 120.74 117.05) (width 0.25) (layer "F.Cu") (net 18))
 (segment (start 122.21 120.19) (end 128.48 120.19) (width 0.25) (layer "F.Cu") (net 18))
 (segment (start 120.74 117.05) (end 121.35 117.66) (width 0.25) (layer "F.Cu") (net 18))
 (segment (start 121.35 119.33) (end 122.21 120.19) (width 0.25) (layer "F.Cu") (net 18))
 (segment (start 129.21 119.46) (end 129.21 117.89) (width 0.25) (layer "F.Cu") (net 18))
 (segment (start 121.35 117.66) (end 121.35 119.33) (width 0.25) (layer "F.Cu") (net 18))
 (via (at 120.02 117.05) (size 0.8) (drill 0.4) (layers "F.Cu" "B.Cu") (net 18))
 (segment (start 120.025 117.055) (end 120.02 117.05) (width 0.25) (layer "B.Cu") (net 18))
 (segment (start 122.3578 117.055) (end 120.025 117.055) (width 0.25) (layer "B.Cu") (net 18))
 (segment (start 134.19 111.3) (end 120.710001 111.3) (width 0.25) (layer "F.Cu") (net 19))
 (segment (start 134.74 111.85) (end 134.19 111.3) (width 0.25) (layer "F.Cu") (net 19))
 (segment (start 134.74 113.4) (end 134.74 111.85) (width 0.25) (layer "F.Cu") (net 19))
 (segment (start 120.710001 111.3) (end 120.040001 111.97) (width 0.25) (layer "F.Cu") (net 19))
 (via (at 120.040001 111.97) (size 0.8) (drill 0.4) (layers "F.Cu" "B.Cu") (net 19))
 (segment (start 120.045001 111.975) (end 120.040001 111.97) (width 0.25) (layer "B.Cu") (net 19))
 (segment (start 122.3578 111.975) (end 120.045001 111.975) (width 0.25) (layer "B.Cu") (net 19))
 (segment (start 141.876 119.27) (end 145.17 119.27) (width 0.25) (layer "B.Cu") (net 23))
 (segment (start 138.535 114.08) (end 140.242 114.08) (width 0.25) (layer "B.Cu") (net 23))
 (segment (start 141.441001 118.835001) (end 141.876 119.27) (width 0.25) (layer "B.Cu") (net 23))
 (segment (start 146.04 118.4) (end 146.04 107.84) (width 0.25) (layer "B.Cu") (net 23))
 (segment (start 145.17 119.27) (end 146.04 118.4) (width 0.25) (layer "B.Cu") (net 23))
 (segment (start 146.04 107.84) (end 144.02 105.82) (width 0.25) (layer "B.Cu") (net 23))
 (segment (start 141.441001 115.279001) (end 141.441001 118.835001) (width 0.25) (layer "B.Cu") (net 23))
 (segment (start 140.242 114.08) (end 141.441001 115.279001) (width 0.25) (layer "B.Cu") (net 23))
 (segment (start 138.55 117.89) (end 140.53 119.87) (width 0.25) (layer "B.Cu") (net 22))
 (segment (start 140.53 119.87) (end 145.47 119.87) (width 0.25) (layer "B.Cu") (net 22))
 (segment (start 145.47 119.87) (end 146.558 118.782) (width 0.25) (layer "B.Cu") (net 22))
 (segment (start 138.535 117.89) (end 138.55 117.89) (width 0.25) (layer "B.Cu") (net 22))
 (segment (start 146.558 105.408) (end 145.605001 104.455001) (width 0.25) (layer "B.Cu") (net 22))
 (segment (start 146.558 118.782) (end 146.558 105.408) (width 0.25) (layer "B.Cu") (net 22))
 (segment (start 142.655001 104.455001) (end 141.48 103.28) (width 0.25) (layer "B.Cu") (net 22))
 (segment (start 145.605001 104.455001) (end 142.655001 104.455001) (width 0.25) (layer "B.Cu") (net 22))
 (segment (start 136.26 105.8) (end 136.26 107.05) (width 0.25) (layer "F.Cu") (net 21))
 (segment (start 136.26 107.05) (end 136.652 107.442) (width 0.25) (layer "F.Cu") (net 21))
 (segment (start 136.652 107.442) (end 140.97 107.442) (width 0.25) (layer "F.Cu") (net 21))
 (segment (start 141.48 106.932) (end 141.48 105.82) (width 0.25) (layer "F.Cu") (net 21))
 (segment (start 140.97 107.442) (end 141.48 106.932) (width 0.25) (layer "F.Cu") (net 21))
 (segment (start 134.56 116.62) (end 135.89 115.29) (width 0.25) (layer "B.Cu") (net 21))
 (segment (start 135.89 106.17) (end 136.26 105.8) (width 0.25) (layer "B.Cu") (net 21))
 (segment (start 133.585 116.62) (end 134.56 116.62) (width 0.25) (layer "B.Cu") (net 21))
 (segment (start 135.89 115.29) (end 135.89 106.17) (width 0.25) (layer "B.Cu") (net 21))
 (segment (start 138.94 107.95) (end 138.94 105.82) (width 0.25) (layer "B.Cu") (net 20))
 (segment (start 136.398 116.332) (end 136.398 110.492) (width 0.25) (layer "B.Cu") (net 20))
 (segment (start 136.398 110.492) (end 138.94 107.95) (width 0.25) (layer "B.Cu") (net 20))
 (segment (start 134.84 117.89) (end 136.398 116.332) (width 0.25) (layer "B.Cu") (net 20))
 (segment (start 133.585 117.89) (end 134.84 117.89) (width 0.25) (layer "B.Cu") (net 20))
 (segment (start 131.352 110.27) (end 135.416 110.27) (width 0.25) (layer "F.Cu") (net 5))
 (segment (start 144.428 103.28) (end 144.02 103.28) (width 0.25) (layer "F.Cu") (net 5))
 (segment (start 134.74 120.23) (end 133.64 121.33) (width 0.25) (layer "F.Cu") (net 5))
 (segment (start 140.178 99.432699) (end 138.502999 99.432699) (width 0.25) (layer "F.Cu") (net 5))
 (segment (start 136.398 116.332) (end 134.83 117.9) (width 0.25) (layer "F.Cu") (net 5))
 (segment (start 138.178002 96.757698) (end 144.777998 96.757698) (width 1) (layer "F.Cu") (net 5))
 (segment (start 135.416 110.27) (end 136.398 111.252) (width 0.25) (layer "F.Cu") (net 5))
 (segment (start 144.777998 96.757698) (end 144.777998 99.107702) (width 1) (layer "F.Cu") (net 5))
 (segment (start 129.21 113.716) (end 133.394 117.9) (width 0.25) (layer "F.Cu") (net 5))
 (segment (start 134.46 120.51) (end 143.93 120.51) (width 0.25) (layer "F.Cu") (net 5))
 (segment (start 144.78 114.046) (end 146.05 114.046) (width 0.25) (layer "F.Cu") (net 5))
 (segment (start 126.41 121.33) (end 125.64 122.1) (width 0.25) (layer "F.Cu") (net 5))
 (segment (start 144.02 99.8657) (end 144.678001 99.207699) (width 0.25) (layer "F.Cu") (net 5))
 (segment (start 143.93 120.51) (end 146.05 118.39) (width 0.25) (layer "F.Cu") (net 5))
 (segment (start 133.64 121.33) (end 134.46 120.51) (width 0.25) (layer "F.Cu") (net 5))
 (segment (start 144.02 99.2437) (end 144.690001 98.573699) (width 0.25) (layer "F.Cu") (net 5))
 (segment (start 138.277999 99.207699) (end 137.053699 99.207699) (width 0.25) (layer "F.Cu") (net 5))
 (segment (start 143.256 108.204) (end 146.05 108.204) (width 0.25) (layer "F.Cu") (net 5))
 (segment (start 146.05 114.046) (end 146.05 108.204) (width 0.25) (layer "F.Cu") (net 5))
 (segment (start 130.12 121.33) (end 126.41 121.33) (width 0.25) (layer "F.Cu") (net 5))
 (segment (start 125.64 122.1) (end 125.64 123.25) (width 0.25) (layer "F.Cu") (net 5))
 (segment (start 144.02 103.28) (end 144.02 99.8657) (width 0.25) (layer "F.Cu") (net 5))
 (segment (start 129.21 113.39) (end 129.21 113.716) (width 0.25) (layer "F.Cu") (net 5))
 (segment (start 146.05 104.902) (end 144.428 103.28) (width 0.25) (layer "F.Cu") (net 5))
 (segment (start 146.05 118.39) (end 146.05 114.046) (width 0.25) (layer "F.Cu") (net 5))
 (segment (start 131.318 110.236) (end 131.352 110.27) (width 0.25) (layer "F.Cu") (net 5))
 (segment (start 136.398 111.252) (end 136.398 116.332) (width 0.25) (layer "F.Cu") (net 5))
 (segment (start 123.698 96.774) (end 122.126 98.346) (width 0.25) (layer "F.Cu") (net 5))
 (segment (start 133.394 117.9) (end 134.74 117.9) (width 0.25) (layer "F.Cu") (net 5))
 (segment (start 138.178002 96.757698) (end 138.178002 99.107702) (width 1) (layer "F.Cu") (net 5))
 (segment (start 134.62 96.774) (end 123.698 96.774) (width 0.25) (layer "F.Cu") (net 5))
 (segment (start 133.64 121.33) (end 130.12 121.33) (width 0.25) (layer "F.Cu") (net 5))
 (segment (start 138.502999 99.432699) (end 138.277999 99.207699) (width 0.25) (layer "F.Cu") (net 5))
 (segment (start 146.05 108.204) (end 146.05 104.902) (width 0.25) (layer "F.Cu") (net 5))
 (segment (start 144.777998 99.107702) (end 144.678001 99.207699) (width 1) (layer "F.Cu") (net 5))
 (segment (start 134.83 117.9) (end 134.74 117.9) (width 0.25) (layer "F.Cu") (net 5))
 (segment (start 138.178002 99.107702) (end 138.277999 99.207699) (width 1) (layer "F.Cu") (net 5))
 (segment (start 134.74 117.9) (end 134.74 120.23) (width 0.25) (layer "F.Cu") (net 5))
 (segment (start 122.126 98.346) (end 122.126 103.554) (width 0.25) (layer "F.Cu") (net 5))
 (segment (start 137.053699 99.207699) (end 134.62 96.774) (width 0.25) (layer "F.Cu") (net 5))
 (via (at 130.12 121.33) (size 0.8) (drill 0.4) (layers "F.Cu" "B.Cu") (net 5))
 (via (at 143.256 108.204) (size 0.8) (drill 0.4) (layers "F.Cu" "B.Cu") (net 5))
 (via (at 144.78 114.046) (size 0.8) (drill 0.4) (layers "F.Cu" "B.Cu") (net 5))
 (via (at 131.318 110.236) (size 0.8) (drill 0.4) (layers "F.Cu" "B.Cu") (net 5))
 (segment (start 144.7738 115.782) (end 144.7738 117.4612) (width 0.25) (layer "B.Cu") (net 5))
 (segment (start 128.4244 117.055) (end 130.12 118.7506) (width 0.25) (layer "B.Cu") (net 5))
 (segment (start 142.865 108.595) (end 143.256 108.204) (width 0.25) (layer "B.Cu") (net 5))
 (segment (start 131.352 110.27) (end 131.318 110.236) (width 0.25) (layer "B.Cu") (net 5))
 (segment (start 142.3862 111.718) (end 142.3862 110.1288) (width 0.25) (layer "B.Cu") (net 5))
 (segment (start 142.865 109.65) (end 142.865 108.595) (width 0.25) (layer "B.Cu") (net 5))
 (segment (start 130.12 118.7506) (end 130.12 121.33) (width 0.25) (layer "B.Cu") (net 5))
 (segment (start 144.7738 115.782) (end 144.7738 114.0522) (width 0.25) (layer "B.Cu") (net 5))
 (segment (start 144.7738 117.4612) (end 144.305 117.93) (width 0.25) (layer "B.Cu") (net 5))
 (segment (start 127.0822 117.055) (end 128.4244 117.055) (width 0.25) (layer "B.Cu") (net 5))
 (segment (start 133.585 110.27) (end 131.352 110.27) (width 0.25) (layer "B.Cu") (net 5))
 (segment (start 144.7738 114.0522) (end 144.78 114.046) (width 0.25) (layer "B.Cu") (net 5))
 (segment (start 142.3862 110.1288) (end 142.865 109.65) (width 0.25) (layer "B.Cu") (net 5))
 (segment (start 142.494 101.346) (end 142.79 101.05) (width 0.25) (layer "F.Cu") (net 10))
 (segment (start 138.94 103.28) (end 138.94 102.106) (width 0.25) (layer "F.Cu") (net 10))
 (segment (start 142.778 101.038) (end 142.79 101.05) (width 0.25) (layer "F.Cu") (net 10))
 (segment (start 139.7 101.346) (end 142.494 101.346) (width 0.25) (layer "F.Cu") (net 10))
 (segment (start 142.778 99.432699) (end 142.778 101.038) (width 0.25) (layer "F.Cu") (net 10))
 (segment (start 138.94 102.106) (end 139.7 101.346) (width 0.25) (layer "F.Cu") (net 10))
 (segment (start 124.24 119.199) (end 124.24 125.88) (width 0.25) (layer "B.Cu") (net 10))
 (segment (start 138.43 125.65) (end 138.43 120.2) (width 0.25) (layer "B.Cu") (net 10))
 (segment (start 136.906 118.676) (end 136.906 110.924) (width 0.25) (layer "B.Cu") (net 10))
 (segment (start 136.906 110.924) (end 137.56 110.27) (width 0.25) (layer "B.Cu") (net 10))
 (segment (start 128.826 103.554) (end 133.680998 103.554) (width 0.25) (layer "B.Cu") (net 10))
 (segment (start 140.208 109.728) (end 140.208 104.548) (width 0.25) (layer "B.Cu") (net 10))
 (segment (start 138.94 102.11) (end 138.94 103.28) (width 0.25) (layer "B.Cu") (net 10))
 (segment (start 138.535 110.27) (end 139.666 110.27) (width 0.25) (layer "B.Cu") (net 10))
 (segment (start 138.2 101.37) (end 138.94 102.11) (width 0.25) (layer "B.Cu") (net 10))
 (segment (start 124.24 125.88) (end 125.99 127.63) (width 0.25) (layer "B.Cu") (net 10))
 (segment (start 125.114 118.325) (end 124.24 119.199) (width 0.25) (layer "B.Cu") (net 10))
 (segment (start 125.99 127.63) (end 136.45 127.63) (width 0.25) (layer "B.Cu") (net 10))
 (segment (start 133.680998 103.554) (end 135.864998 101.37) (width 0.25) (layer "B.Cu") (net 10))
 (segment (start 137.56 110.27) (end 138.535 110.27) (width 0.25) (layer "B.Cu") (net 10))
 (segment (start 135.864998 101.37) (end 138.2 101.37) (width 0.25) (layer "B.Cu") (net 10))
 (segment (start 140.208 104.548) (end 138.94 103.28) (width 0.25) (layer "B.Cu") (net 10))
 (segment (start 139.666 110.27) (end 140.208 109.728) (width 0.25) (layer "B.Cu") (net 10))
 (segment (start 136.45 127.63) (end 138.43 125.65) (width 0.25) (layer "B.Cu") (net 10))
 (segment (start 127.0822 118.325) (end 125.114 118.325) (width 0.25) (layer "B.Cu") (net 10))
 (segment (start 138.43 120.2) (end 136.906 118.676) (width 0.25) (layer "B.Cu") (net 10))
 (segment (start 132.8 114.08) (end 133.585 114.08) (width 0.25) (layer "B.Cu") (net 31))
 (segment (start 127.0822 109.435) (end 128.155 109.435) (width 0.25) (layer "B.Cu") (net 31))
 (segment (start 128.155 109.435) (end 132.8 114.08) (width 0.25) (layer "B.Cu") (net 31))
 (segment (start 134.88501 114.426758) (end 134.88501 113.04101) (width 0.25) (layer "B.Cu") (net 32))
 (segment (start 134.654 112.81) (end 133.585 112.81) (width 0.25) (layer "B.Cu") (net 32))
 (segment (start 134.606758 114.70501) (end 134.88501 114.426758) (width 0.25) (layer "B.Cu") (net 32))
 (segment (start 128.563232 110.705) (end 132.563242 114.70501) (width 0.25) (layer "B.Cu") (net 32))
 (segment (start 132.563242 114.70501) (end 134.606758 114.70501) (width 0.25) (layer "B.Cu") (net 32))
 (segment (start 127.0822 110.705) (end 128.563232 110.705) (width 0.25) (layer "B.Cu") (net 32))
 (segment (start 134.88501 113.04101) (end 134.654 112.81) (width 0.25) (layer "B.Cu") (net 32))
 (segment (start 125.68 108.46) (end 128.272 108.46) (width 0.25) (layer "B.Cu") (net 34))
 (segment (start 127.0822 113.245) (end 125.74 113.245) (width 0.25) (layer "B.Cu") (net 34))
 (segment (start 125.74 113.245) (end 125.15 112.655) (width 0.25) (layer "B.Cu") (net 34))
 (segment (start 125.15 108.99) (end 125.68 108.46) (width 0.25) (layer "B.Cu") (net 34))
 (segment (start 125.15 112.655) (end 125.15 108.99) (width 0.25) (layer "B.Cu") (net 34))
 (segment (start 128.272 108.46) (end 131.352 111.54) (width 0.25) (layer "B.Cu") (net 34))
 (segment (start 131.352 111.54) (end 133.585 111.54) (width 0.25) (layer "B.Cu") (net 34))
 (segment (start 133.585 115.35) (end 134.598178 115.35) (width 0.25) (layer "B.Cu") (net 24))
 (segment (start 134.598178 115.35) (end 135.40997 114.538208) (width 0.25) (layer "B.Cu") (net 24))
 (segment (start 135.40997 114.538208) (end 135.40997 108.29997) (width 0.25) (layer "B.Cu") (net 24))
 (segment (start 134.4 104.15) (end 135.29 103.26) (width 0.25) (layer "B.Cu") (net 24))
 (segment (start 135.29 103.26) (end 136.26 103.26) (width 0.25) (layer "B.Cu") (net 24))
 (segment (start 134.4 107.29) (end 134.4 104.15) (width 0.25) (layer "B.Cu") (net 24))
 (segment (start 135.40997 108.29997) (end 134.4 107.29) (width 0.25) (layer "B.Cu") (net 24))
 (segment (start 144.415 109.65) (end 144.415 111.3592) (width 0.25) (layer "B.Cu") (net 29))
 (segment (start 138.535 111.54) (end 139.7 111.54) (width 0.25) (layer "B.Cu") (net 29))
 (segment (start 139.601008 111.54) (end 138.535 111.54) (width 0.25) (layer "B.Cu") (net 29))
 (segment (start 139.7 111.54) (end 141.55 113.39) (width 0.25) (layer "B.Cu") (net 29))
 (segment (start 144.7738 112.7262) (end 144.7738 111.718) (width 0.25) (layer "B.Cu") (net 29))
 (segment (start 144.11 113.39) (end 144.7738 112.7262) (width 0.25) (layer "B.Cu") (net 29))
 (segment (start 141.55 113.39) (end 144.11 113.39) (width 0.25) (layer "B.Cu") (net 29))
 (segment (start 144.415 111.3592) (end 144.7738 111.718) (width 0.25) (layer "B.Cu") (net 29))
 (segment (start 138.535 112.81) (end 139.86 112.81) (width 0.25) (layer "B.Cu") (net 30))
 (segment (start 139.86 112.81) (end 142.3862 115.3362) (width 0.25) (layer "B.Cu") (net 30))
 (segment (start 142.3862 115.3362) (end 142.3862 115.782) (width 0.25) (layer "B.Cu") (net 30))
 (segment (start 139.4159 112.81) (end 138.535 112.81) (width 0.25) (layer "B.Cu") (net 30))
 (segment (start 142.755 117.93) (end 142.755 116.1508) (width 0.25) (layer "B.Cu") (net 30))
 (segment (start 142.755 116.1508) (end 142.3862 115.782) (width 0.25) (layer "B.Cu") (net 30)))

